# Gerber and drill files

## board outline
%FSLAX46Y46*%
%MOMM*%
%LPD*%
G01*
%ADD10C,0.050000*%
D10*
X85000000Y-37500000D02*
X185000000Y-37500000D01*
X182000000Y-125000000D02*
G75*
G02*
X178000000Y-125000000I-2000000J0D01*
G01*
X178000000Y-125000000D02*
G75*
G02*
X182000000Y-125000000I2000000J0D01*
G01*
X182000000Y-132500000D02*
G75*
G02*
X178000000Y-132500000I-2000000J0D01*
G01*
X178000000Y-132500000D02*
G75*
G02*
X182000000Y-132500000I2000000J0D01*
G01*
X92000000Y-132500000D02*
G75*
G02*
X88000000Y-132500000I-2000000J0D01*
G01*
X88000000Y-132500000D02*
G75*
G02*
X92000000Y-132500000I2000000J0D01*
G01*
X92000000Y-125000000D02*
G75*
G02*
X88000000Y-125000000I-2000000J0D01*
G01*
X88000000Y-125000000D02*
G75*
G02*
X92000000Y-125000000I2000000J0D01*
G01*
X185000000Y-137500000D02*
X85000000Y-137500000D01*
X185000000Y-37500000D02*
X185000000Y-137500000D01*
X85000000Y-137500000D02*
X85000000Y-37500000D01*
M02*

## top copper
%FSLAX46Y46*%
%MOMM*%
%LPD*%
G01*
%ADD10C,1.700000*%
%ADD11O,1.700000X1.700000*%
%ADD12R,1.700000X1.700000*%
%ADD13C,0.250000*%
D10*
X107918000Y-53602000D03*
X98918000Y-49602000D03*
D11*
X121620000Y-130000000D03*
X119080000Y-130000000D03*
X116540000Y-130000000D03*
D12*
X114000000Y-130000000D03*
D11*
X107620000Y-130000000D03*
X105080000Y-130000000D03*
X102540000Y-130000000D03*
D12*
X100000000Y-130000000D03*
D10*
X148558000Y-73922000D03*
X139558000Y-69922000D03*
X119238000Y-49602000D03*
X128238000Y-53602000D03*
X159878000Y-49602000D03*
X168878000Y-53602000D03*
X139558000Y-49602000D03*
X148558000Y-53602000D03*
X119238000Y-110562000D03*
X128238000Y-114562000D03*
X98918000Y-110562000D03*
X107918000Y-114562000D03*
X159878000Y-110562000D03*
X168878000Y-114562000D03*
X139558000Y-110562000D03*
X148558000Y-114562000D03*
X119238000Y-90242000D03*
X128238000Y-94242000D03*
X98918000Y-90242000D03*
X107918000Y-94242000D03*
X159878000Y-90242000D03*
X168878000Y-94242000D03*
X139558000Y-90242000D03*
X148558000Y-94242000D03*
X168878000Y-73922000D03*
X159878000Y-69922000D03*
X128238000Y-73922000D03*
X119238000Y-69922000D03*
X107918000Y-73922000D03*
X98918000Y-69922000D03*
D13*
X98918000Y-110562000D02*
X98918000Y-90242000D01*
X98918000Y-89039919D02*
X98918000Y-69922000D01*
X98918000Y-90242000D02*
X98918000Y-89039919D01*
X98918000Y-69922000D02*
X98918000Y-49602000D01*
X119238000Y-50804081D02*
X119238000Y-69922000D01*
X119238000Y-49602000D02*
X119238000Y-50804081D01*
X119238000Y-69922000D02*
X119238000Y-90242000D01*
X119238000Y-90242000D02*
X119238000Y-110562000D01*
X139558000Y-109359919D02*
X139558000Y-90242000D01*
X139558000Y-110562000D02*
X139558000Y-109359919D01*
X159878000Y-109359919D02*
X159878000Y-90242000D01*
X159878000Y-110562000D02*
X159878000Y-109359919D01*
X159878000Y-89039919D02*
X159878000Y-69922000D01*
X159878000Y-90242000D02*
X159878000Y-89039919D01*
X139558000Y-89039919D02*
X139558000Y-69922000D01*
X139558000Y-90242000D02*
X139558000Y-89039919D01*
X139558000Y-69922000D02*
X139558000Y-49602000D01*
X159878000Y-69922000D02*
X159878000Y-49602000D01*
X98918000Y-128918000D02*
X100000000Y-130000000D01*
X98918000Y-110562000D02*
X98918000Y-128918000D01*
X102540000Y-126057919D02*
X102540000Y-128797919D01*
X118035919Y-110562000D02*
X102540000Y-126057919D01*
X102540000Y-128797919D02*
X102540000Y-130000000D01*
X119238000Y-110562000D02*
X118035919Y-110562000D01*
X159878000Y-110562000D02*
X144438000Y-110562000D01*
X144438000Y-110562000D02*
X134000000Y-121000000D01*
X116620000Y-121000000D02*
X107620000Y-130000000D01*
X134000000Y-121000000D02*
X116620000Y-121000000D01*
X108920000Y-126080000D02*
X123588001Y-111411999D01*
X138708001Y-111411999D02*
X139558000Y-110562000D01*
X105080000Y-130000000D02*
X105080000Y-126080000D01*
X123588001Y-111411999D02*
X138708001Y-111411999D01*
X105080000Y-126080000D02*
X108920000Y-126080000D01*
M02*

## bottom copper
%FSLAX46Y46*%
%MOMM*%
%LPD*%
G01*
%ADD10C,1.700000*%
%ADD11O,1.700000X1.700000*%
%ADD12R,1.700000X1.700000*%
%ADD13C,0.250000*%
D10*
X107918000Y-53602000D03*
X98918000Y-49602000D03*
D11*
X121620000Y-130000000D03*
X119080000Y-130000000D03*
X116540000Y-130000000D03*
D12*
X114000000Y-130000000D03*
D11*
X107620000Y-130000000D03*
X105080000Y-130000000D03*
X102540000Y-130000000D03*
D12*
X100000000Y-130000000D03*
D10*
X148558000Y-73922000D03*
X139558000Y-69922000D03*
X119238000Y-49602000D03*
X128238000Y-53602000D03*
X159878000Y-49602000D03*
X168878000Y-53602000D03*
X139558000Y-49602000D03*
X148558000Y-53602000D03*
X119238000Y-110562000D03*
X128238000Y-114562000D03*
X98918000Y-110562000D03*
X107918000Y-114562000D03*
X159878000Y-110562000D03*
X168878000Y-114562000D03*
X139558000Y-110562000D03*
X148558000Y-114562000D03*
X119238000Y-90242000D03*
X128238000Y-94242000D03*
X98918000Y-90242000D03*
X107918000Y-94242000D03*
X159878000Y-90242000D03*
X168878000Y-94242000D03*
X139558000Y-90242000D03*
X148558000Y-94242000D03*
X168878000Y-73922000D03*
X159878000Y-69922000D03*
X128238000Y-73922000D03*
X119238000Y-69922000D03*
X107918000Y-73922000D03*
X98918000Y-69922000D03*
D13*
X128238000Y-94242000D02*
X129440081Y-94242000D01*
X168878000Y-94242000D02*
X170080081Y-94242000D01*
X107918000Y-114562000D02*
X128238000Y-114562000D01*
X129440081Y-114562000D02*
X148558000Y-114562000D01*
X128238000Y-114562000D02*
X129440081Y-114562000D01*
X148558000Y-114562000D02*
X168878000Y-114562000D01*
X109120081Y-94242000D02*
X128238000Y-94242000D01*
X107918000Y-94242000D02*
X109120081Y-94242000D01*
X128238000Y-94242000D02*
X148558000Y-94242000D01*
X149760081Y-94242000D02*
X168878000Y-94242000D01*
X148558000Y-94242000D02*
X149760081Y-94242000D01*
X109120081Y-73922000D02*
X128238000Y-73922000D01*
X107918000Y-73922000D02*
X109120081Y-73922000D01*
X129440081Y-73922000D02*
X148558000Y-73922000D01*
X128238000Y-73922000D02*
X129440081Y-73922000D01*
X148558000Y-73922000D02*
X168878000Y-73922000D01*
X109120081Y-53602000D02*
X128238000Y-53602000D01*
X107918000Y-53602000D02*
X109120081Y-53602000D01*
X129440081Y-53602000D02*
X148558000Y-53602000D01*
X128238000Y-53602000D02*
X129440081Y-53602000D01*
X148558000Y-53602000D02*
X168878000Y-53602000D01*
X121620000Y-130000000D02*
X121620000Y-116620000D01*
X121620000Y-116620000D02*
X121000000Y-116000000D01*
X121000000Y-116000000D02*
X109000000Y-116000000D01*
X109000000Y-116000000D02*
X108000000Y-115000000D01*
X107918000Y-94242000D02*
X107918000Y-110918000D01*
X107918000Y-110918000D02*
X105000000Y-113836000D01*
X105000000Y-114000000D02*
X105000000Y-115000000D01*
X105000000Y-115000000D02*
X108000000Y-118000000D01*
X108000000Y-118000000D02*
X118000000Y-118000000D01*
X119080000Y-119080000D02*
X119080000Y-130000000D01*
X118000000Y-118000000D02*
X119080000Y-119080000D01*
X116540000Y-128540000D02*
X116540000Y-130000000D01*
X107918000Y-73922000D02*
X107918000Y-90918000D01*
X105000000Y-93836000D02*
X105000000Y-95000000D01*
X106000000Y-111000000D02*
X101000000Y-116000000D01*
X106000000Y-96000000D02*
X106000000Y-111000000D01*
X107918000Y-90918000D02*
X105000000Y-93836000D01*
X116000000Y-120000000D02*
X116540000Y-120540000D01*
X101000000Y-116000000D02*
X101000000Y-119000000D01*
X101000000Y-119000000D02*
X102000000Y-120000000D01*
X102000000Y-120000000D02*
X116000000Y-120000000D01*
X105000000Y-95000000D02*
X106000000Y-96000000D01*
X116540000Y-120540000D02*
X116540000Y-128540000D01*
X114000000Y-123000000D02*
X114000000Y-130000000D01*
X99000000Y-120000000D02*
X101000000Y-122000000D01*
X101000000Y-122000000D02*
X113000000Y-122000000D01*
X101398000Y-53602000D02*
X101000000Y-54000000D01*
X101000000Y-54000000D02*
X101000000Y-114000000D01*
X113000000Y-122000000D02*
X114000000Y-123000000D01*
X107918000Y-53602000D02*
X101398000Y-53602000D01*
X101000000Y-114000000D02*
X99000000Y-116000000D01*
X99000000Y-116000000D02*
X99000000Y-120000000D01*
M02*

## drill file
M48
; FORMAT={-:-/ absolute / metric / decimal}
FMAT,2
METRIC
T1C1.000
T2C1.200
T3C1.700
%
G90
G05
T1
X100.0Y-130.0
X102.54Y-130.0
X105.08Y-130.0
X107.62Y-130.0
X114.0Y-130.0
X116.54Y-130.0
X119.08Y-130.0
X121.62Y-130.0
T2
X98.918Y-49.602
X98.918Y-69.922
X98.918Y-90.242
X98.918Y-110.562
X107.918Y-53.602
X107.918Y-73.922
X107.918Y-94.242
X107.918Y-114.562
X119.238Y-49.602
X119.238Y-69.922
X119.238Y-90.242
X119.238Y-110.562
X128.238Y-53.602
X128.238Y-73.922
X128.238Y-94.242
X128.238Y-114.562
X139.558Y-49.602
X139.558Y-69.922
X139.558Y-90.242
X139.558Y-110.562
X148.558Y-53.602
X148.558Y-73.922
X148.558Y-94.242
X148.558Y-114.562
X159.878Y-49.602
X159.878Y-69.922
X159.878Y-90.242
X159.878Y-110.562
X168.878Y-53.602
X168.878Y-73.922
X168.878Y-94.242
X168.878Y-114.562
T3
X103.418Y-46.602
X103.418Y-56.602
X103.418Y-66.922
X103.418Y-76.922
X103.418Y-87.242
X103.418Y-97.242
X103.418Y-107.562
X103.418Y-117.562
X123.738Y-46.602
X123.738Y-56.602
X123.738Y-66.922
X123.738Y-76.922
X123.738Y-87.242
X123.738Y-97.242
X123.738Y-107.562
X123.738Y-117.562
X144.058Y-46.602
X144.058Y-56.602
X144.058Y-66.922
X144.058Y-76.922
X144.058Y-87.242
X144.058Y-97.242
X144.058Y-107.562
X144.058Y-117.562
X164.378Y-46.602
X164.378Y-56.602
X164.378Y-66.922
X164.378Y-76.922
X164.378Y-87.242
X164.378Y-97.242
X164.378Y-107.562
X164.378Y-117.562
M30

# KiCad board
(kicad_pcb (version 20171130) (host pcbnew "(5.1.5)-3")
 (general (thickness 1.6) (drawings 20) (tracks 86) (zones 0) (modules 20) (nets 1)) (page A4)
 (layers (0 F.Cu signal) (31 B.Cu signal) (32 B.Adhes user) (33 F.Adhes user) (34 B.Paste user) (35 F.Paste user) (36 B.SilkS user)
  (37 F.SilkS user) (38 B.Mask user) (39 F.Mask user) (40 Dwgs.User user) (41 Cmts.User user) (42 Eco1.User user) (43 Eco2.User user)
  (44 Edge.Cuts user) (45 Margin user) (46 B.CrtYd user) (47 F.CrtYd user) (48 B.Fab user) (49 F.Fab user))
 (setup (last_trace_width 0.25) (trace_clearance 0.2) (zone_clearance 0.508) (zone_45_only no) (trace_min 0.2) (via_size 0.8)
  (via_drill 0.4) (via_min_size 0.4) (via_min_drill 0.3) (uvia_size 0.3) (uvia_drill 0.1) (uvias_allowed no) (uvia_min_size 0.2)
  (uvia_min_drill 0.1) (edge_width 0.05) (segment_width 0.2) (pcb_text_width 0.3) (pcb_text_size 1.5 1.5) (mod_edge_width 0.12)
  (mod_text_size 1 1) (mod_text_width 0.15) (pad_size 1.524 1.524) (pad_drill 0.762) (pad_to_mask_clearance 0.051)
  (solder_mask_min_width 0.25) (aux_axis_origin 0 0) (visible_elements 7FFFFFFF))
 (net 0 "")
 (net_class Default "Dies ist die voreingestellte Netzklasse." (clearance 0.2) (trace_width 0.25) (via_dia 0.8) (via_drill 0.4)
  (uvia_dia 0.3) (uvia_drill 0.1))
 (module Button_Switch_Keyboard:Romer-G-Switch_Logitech (layer F.Cu) (at 103.418 51.602)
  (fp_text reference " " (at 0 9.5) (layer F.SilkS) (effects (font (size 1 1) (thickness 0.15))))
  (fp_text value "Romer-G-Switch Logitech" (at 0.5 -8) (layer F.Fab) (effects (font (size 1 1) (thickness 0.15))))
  (pad "" np_thru_hole circle (at 0 5) (size 1.7 1.7) (drill 1.7) (layers *.Cu *.Mask))
  (pad "" np_thru_hole circle (at 0 -5) (size 1.7 1.7) (drill 1.7) (layers *.Cu *.Mask))
  (pad 2 thru_hole circle (at 4.5 2) (size 1.7 1.7) (drill 1.2) (layers *.Cu *.Mask))
  (pad 1 thru_hole circle (at -4.5 -2) (size 1.7 1.7) (drill 1.2) (layers *.Cu *.Mask)))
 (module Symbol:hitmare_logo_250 (layer B.Cu) (at 134 82 180)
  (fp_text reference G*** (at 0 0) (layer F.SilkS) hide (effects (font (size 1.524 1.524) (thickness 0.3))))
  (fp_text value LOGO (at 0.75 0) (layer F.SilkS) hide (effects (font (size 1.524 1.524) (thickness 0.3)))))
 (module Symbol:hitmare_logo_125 (layer F.Cu) (at 180 46)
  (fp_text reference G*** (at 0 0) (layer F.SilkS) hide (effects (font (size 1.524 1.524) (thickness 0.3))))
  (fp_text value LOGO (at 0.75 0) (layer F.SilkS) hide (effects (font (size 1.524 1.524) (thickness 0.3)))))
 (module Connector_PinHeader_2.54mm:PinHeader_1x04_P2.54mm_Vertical (layer F.Cu) (at 114 130 90)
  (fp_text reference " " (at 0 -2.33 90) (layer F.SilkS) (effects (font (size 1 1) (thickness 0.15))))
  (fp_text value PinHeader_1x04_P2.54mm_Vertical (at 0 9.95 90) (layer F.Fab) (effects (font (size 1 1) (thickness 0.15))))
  (pad 4 thru_hole oval (at 0 7.62 90) (size 1.7 1.7) (drill 1) (layers *.Cu *.Mask))
  (pad 3 thru_hole oval (at 0 5.08 90) (size 1.7 1.7) (drill 1) (layers *.Cu *.Mask))
  (pad 2 thru_hole oval (at 0 2.54 90) (size 1.7 1.7) (drill 1) (layers *.Cu *.Mask))
  (pad 1 thru_hole rect (at 0 0 90) (size 1.7 1.7) (drill 1) (layers *.Cu *.Mask)))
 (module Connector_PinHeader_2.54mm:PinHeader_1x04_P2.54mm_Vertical (layer F.Cu) (at 100 130 90)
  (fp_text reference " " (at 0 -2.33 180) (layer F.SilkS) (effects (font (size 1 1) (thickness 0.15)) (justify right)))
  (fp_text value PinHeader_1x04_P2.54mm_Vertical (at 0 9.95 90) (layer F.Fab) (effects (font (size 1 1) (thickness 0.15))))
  (pad 4 thru_hole oval (at 0 7.62 90) (size 1.7 1.7) (drill 1) (layers *.Cu *.Mask))
  (pad 3 thru_hole oval (at 0 5.08 90) (size 1.7 1.7) (drill 1) (layers *.Cu *.Mask))
  (pad 2 thru_hole oval (at 0 2.54 90) (size 1.7 1.7) (drill 1) (layers *.Cu *.Mask))
  (pad 1 thru_hole rect (at 0 0 90) (size 1.7 1.7) (drill 1) (layers *.Cu *.Mask)))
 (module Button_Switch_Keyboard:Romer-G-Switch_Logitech (layer F.Cu) (at 144.058 71.922)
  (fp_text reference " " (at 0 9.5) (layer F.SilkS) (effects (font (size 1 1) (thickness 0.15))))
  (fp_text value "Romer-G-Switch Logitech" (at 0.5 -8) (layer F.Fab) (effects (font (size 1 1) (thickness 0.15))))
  (pad "" np_thru_hole circle (at 0 5) (size 1.7 1.7) (drill 1.7) (layers *.Cu *.Mask))
  (pad "" np_thru_hole circle (at 0 -5) (size 1.7 1.7) (drill 1.7) (layers *.Cu *.Mask))
  (pad 2 thru_hole circle (at 4.5 2) (size 1.7 1.7) (drill 1.2) (layers *.Cu *.Mask))
  (pad 1 thru_hole circle (at -4.5 -2) (size 1.7 1.7) (drill 1.2) (layers *.Cu *.Mask)))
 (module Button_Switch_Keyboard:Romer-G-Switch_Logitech (layer F.Cu) (at 123.738 51.602)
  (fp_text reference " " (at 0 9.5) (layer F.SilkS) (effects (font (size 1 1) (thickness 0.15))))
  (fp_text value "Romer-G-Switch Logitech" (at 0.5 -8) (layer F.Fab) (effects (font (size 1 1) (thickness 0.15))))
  (pad 1 thru_hole circle (at -4.5 -2) (size 1.7 1.7) (drill 1.2) (layers *.Cu *.Mask))
  (pad 2 thru_hole circle (at 4.5 2) (size 1.7 1.7) (drill 1.2) (layers *.Cu *.Mask))
  (pad "" np_thru_hole circle (at 0 -5) (size 1.7 1.7) (drill 1.7) (layers *.Cu *.Mask))
  (pad "" np_thru_hole circle (at 0 5) (size 1.7 1.7) (drill 1.7) (layers *.Cu *.Mask)))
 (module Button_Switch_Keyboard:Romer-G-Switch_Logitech (layer F.Cu) (at 164.378 51.602)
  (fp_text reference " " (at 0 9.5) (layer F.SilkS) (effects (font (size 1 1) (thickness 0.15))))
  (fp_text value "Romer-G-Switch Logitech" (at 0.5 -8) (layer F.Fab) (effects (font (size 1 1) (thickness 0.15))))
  (pad 1 thru_hole circle (at -4.5 -2) (size 1.7 1.7) (drill 1.2) (layers *.Cu *.Mask))
  (pad 2 thru_hole circle (at 4.5 2) (size 1.7 1.7) (drill 1.2) (layers *.Cu *.Mask))
  (pad "" np_thru_hole circle (at 0 -5) (size 1.7 1.7) (drill 1.7) (layers *.Cu *.Mask))
  (pad "" np_thru_hole circle (at 0 5) (size 1.7 1.7) (drill 1.7) (layers *.Cu *.Mask)))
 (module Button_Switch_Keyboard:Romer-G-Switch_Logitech (layer F.Cu) (at 144.058 51.602)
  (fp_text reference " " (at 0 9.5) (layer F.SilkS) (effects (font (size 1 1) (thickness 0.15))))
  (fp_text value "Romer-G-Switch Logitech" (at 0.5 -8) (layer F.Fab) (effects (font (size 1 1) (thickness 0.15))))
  (pad 1 thru_hole circle (at -4.5 -2) (size 1.7 1.7) (drill 1.2) (layers *.Cu *.Mask))
  (pad 2 thru_hole circle (at 4.5 2) (size 1.7 1.7) (drill 1.2) (layers *.Cu *.Mask))
  (pad "" np_thru_hole circle (at 0 -5) (size 1.7 1.7) (drill 1.7) (layers *.Cu *.Mask))
  (pad "" np_thru_hole circle (at 0 5) (size 1.7 1.7) (drill 1.7) (layers *.Cu *.Mask)))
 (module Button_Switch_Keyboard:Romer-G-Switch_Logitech (layer F.Cu) (at 123.738 112.562)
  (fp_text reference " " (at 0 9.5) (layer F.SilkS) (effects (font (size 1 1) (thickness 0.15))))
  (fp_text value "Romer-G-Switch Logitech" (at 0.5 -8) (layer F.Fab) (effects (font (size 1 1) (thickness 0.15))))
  (pad 1 thru_hole circle (at -4.5 -2) (size 1.7 1.7) (drill 1.2) (layers *.Cu *.Mask))
  (pad 2 thru_hole circle (at 4.5 2) (size 1.7 1.7) (drill 1.2) (layers *.Cu *.Mask))
  (pad "" np_thru_hole circle (at 0 -5) (size 1.7 1.7) (drill 1.7) (layers *.Cu *.Mask))
  (pad "" np_thru_hole circle (at 0 5) (size 1.7 1.7) (drill 1.7) (layers *.Cu *.Mask)))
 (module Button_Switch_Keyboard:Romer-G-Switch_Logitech (layer F.Cu) (at 103.418 112.562)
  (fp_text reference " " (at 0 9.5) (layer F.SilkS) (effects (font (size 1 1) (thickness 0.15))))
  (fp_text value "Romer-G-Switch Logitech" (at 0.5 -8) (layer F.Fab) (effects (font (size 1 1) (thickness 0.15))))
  (pad 1 thru_hole circle (at -4.5 -2) (size 1.7 1.7) (drill 1.2) (layers *.Cu *.Mask))
  (pad 2 thru_hole circle (at 4.5 2) (size 1.7 1.7) (drill 1.2) (layers *.Cu *.Mask))
  (pad "" np_thru_hole circle (at 0 -5) (size 1.7 1.7) (drill 1.7) (layers *.Cu *.Mask))
  (pad "" np_thru_hole circle (at 0 5) (size 1.7 1.7) (drill 1.7) (layers *.Cu *.Mask)))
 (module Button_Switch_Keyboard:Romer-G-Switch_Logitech (layer F.Cu) (at 164.378 112.562)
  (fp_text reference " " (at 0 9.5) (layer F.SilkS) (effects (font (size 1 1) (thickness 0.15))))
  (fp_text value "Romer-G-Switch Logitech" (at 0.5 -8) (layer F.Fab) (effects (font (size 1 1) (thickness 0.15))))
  (pad 1 thru_hole circle (at -4.5 -2) (size 1.7 1.7) (drill 1.2) (layers *.Cu *.Mask))
  (pad 2 thru_hole circle (at 4.5 2) (size 1.7 1.7) (drill 1.2) (layers *.Cu *.Mask))
  (pad "" np_thru_hole circle (at 0 -5) (size 1.7 1.7) (drill 1.7) (layers *.Cu *.Mask))
  (pad "" np_thru_hole circle (at 0 5) (size 1.7 1.7) (drill 1.7) (layers *.Cu *.Mask)))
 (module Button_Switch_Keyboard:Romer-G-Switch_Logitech (layer F.Cu) (at 144.058 112.562)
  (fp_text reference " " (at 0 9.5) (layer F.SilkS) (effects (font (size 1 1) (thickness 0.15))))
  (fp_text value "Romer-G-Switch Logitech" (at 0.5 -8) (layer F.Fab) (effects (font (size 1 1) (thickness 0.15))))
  (pad 1 thru_hole circle (at -4.5 -2) (size 1.7 1.7) (drill 1.2) (layers *.Cu *.Mask))
  (pad 2 thru_hole circle (at 4.5 2) (size 1.7 1.7) (drill 1.2) (layers *.Cu *.Mask))
  (pad "" np_thru_hole circle (at 0 -5) (size 1.7 1.7) (drill 1.7) (layers *.Cu *.Mask))
  (pad "" np_thru_hole circle (at 0 5) (size 1.7 1.7) (drill 1.7) (layers *.Cu *.Mask)))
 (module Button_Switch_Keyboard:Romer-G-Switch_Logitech (layer F.Cu) (at 123.738 92.242)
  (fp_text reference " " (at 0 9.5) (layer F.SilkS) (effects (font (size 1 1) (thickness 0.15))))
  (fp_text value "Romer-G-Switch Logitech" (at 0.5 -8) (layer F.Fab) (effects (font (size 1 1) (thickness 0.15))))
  (pad 1 thru_hole circle (at -4.5 -2) (size 1.7 1.7) (drill 1.2) (layers *.Cu *.Mask))
  (pad 2 thru_hole circle (at 4.5 2) (size 1.7 1.7) (drill 1.2) (layers *.Cu *.Mask))
  (pad "" np_thru_hole circle (at 0 -5) (size 1.7 1.7) (drill 1.7) (layers *.Cu *.Mask))
  (pad "" np_thru_hole circle (at 0 5) (size 1.7 1.7) (drill 1.7) (layers *.Cu *.Mask)))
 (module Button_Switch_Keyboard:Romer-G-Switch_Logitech (layer F.Cu) (at 103.418 92.242)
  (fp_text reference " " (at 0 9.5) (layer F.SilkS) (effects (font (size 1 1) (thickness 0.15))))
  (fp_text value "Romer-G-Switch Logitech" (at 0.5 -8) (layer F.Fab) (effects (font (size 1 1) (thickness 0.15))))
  (pad 1 thru_hole circle (at -4.5 -2) (size 1.7 1.7) (drill 1.2) (layers *.Cu *.Mask))
  (pad 2 thru_hole circle (at 4.5 2) (size 1.7 1.7) (drill 1.2) (layers *.Cu *.Mask))
  (pad "" np_thru_hole circle (at 0 -5) (size 1.7 1.7) (drill 1.7) (layers *.Cu *.Mask))
  (pad "" np_thru_hole circle (at 0 5) (size 1.7 1.7) (drill 1.7) (layers *.Cu *.Mask)))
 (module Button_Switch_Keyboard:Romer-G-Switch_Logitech (layer F.Cu) (at 164.378 92.242)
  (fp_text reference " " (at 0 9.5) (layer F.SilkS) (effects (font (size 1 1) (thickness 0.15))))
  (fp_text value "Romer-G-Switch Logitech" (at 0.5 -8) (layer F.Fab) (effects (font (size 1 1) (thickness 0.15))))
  (pad 1 thru_hole circle (at -4.5 -2) (size 1.7 1.7) (drill 1.2) (layers *.Cu *.Mask))
  (pad 2 thru_hole circle (at 4.5 2) (size 1.7 1.7) (drill 1.2) (layers *.Cu *.Mask))
  (pad "" np_thru_hole circle (at 0 -5) (size 1.7 1.7) (drill 1.7) (layers *.Cu *.Mask))
  (pad "" np_thru_hole circle (at 0 5) (size 1.7 1.7) (drill 1.7) (layers *.Cu *.Mask)))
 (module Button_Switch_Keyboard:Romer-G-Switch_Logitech (layer F.Cu) (at 144.058 92.242)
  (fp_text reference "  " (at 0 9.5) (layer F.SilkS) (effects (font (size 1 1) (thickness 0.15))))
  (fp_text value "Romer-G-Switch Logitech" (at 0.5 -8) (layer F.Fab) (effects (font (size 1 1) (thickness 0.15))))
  (pad 1 thru_hole circle (at -4.5 -2) (size 1.7 1.7) (drill 1.2) (layers *.Cu *.Mask))
  (pad 2 thru_hole circle (at 4.5 2) (size 1.7 1.7) (drill 1.2) (layers *.Cu *.Mask))
  (pad "" np_thru_hole circle (at 0 -5) (size 1.7 1.7) (drill 1.7) (layers *.Cu *.Mask))
  (pad "" np_thru_hole circle (at 0 5) (size 1.7 1.7) (drill 1.7) (layers *.Cu *.Mask)))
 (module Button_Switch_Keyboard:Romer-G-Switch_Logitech (layer F.Cu) (at 164.378 71.922)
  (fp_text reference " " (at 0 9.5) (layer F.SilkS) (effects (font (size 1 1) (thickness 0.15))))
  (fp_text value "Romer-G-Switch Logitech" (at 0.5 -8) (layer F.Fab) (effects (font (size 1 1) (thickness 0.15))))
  (pad "" np_thru_hole circle (at 0 5) (size 1.7 1.7) (drill 1.7) (layers *.Cu *.Mask))
  (pad "" np_thru_hole circle (at 0 -5) (size 1.7 1.7) (drill 1.7) (layers *.Cu *.Mask))
  (pad 2 thru_hole circle (at 4.5 2) (size 1.7 1.7) (drill 1.2) (layers *.Cu *.Mask))
  (pad 1 thru_hole circle (at -4.5 -2) (size 1.7 1.7) (drill 1.2) (layers *.Cu *.Mask)))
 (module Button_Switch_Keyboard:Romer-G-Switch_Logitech (layer F.Cu) (at 123.738 71.922)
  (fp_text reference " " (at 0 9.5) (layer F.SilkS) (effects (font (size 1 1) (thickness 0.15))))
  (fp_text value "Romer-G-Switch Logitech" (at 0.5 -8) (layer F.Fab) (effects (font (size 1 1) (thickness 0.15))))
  (pad "" np_thru_hole circle (at 0 5) (size 1.7 1.7) (drill 1.7) (layers *.Cu *.Mask))
  (pad "" np_thru_hole circle (at 0 -5) (size 1.7 1.7) (drill 1.7) (layers *.Cu *.Mask))
  (pad 2 thru_hole circle (at 4.5 2) (size 1.7 1.7) (drill 1.2) (layers *.Cu *.Mask))
  (pad 1 thru_hole circle (at -4.5 -2) (size 1.7 1.7) (drill 1.2) (layers *.Cu *.Mask)))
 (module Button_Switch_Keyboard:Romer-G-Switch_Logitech (layer F.Cu) (at 103.418 71.922)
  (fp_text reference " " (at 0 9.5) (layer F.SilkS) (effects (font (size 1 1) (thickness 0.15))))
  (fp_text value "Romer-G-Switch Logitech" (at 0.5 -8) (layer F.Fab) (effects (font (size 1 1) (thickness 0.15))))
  (pad "" np_thru_hole circle (at 0 5) (size 1.7 1.7) (drill 1.7) (layers *.Cu *.Mask))
  (pad "" np_thru_hole circle (at 0 -5) (size 1.7 1.7) (drill 1.7) (layers *.Cu *.Mask))
  (pad 2 thru_hole circle (at 4.5 2) (size 1.7 1.7) (drill 1.2) (layers *.Cu *.Mask))
  (pad 1 thru_hole circle (at -4.5 -2) (size 1.7 1.7) (drill 1.2) (layers *.Cu *.Mask)))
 (gr_line (start 85 37.5) (end 185 37.5) (layer Edge.Cuts) (width 0.05))
 (gr_circle (center 180 125) (end 182 125) (layer Edge.Cuts) (width 0.05))
 (gr_circle (center 180 132.5) (end 182 132.5) (layer Edge.Cuts) (width 0.05))
 (gr_circle (center 90 132.5) (end 92 132.5) (layer Edge.Cuts) (width 0.05))
 (gr_circle (center 90 125) (end 92 125) (layer Edge.Cuts) (width 0.05))
 (gr_line (start 185 137.5) (end 85 137.5) (layer Edge.Cuts) (width 0.05))
 (gr_line (start 185 37.5) (end 185 137.5) (layer Edge.Cuts) (width 0.05))
 (gr_line (start 85 137.5) (end 85 37.5) (layer Edge.Cuts) (width 0.05))
 (segment (start 128.238 94.242) (end 129.440081 94.242) (width 0.25) (layer B.Cu) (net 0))
 (segment (start 168.878 94.242) (end 170.080081 94.242) (width 0.25) (layer B.Cu) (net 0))
 (segment (start 98.918 110.562) (end 98.918 90.242) (width 0.25) (layer F.Cu) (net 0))
 (segment (start 98.918 89.039919) (end 98.918 69.922) (width 0.25) (layer F.Cu) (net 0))
 (segment (start 98.918 90.242) (end 98.918 89.039919) (width 0.25) (layer F.Cu) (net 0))
 (segment (start 98.918 69.922) (end 98.918 49.602) (width 0.25) (layer F.Cu) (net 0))
 (segment (start 119.238 50.804081) (end 119.238 69.922) (width 0.25) (layer F.Cu) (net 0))
 (segment (start 119.238 49.602) (end 119.238 50.804081) (width 0.25) (layer F.Cu) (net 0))
 (segment (start 119.238 69.922) (end 119.238 90.242) (width 0.25) (layer F.Cu) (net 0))
 (segment (start 119.238 90.242) (end 119.238 110.562) (width 0.25) (layer F.Cu) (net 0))
 (segment (start 139.558 109.359919) (end 139.558 90.242) (width 0.25) (layer F.Cu) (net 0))
 (segment (start 139.558 110.562) (end 139.558 109.359919) (width 0.25) (layer F.Cu) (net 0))
 (segment (start 159.878 109.359919) (end 159.878 90.242) (width 0.25) (layer F.Cu) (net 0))
 (segment (start 159.878 110.562) (end 159.878 109.359919) (width 0.25) (layer F.Cu) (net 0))
 (segment (start 159.878 89.039919) (end 159.878 69.922) (width 0.25) (layer F.Cu) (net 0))
 (segment (start 159.878 90.242) (end 159.878 89.039919) (width 0.25) (layer F.Cu) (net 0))
 (segment (start 139.558 89.039919) (end 139.558 69.922) (width 0.25) (layer F.Cu) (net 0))
 (segment (start 139.558 90.242) (end 139.558 89.039919) (width 0.25) (layer F.Cu) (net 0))
 (segment (start 139.558 69.922) (end 139.558 49.602) (width 0.25) (layer F.Cu) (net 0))
 (segment (start 159.878 69.922) (end 159.878 49.602) (width 0.25) (layer F.Cu) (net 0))
 (segment (start 107.918 114.562) (end 128.238 114.562) (width 0.25) (layer B.Cu) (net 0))
 (segment (start 129.440081 114.562) (end 148.558 114.562) (width 0.25) (layer B.Cu) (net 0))
 (segment (start 128.238 114.562) (end 129.440081 114.562) (width 0.25) (layer B.Cu) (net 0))
 (segment (start 148.558 114.562) (end 168.878 114.562) (width 0.25) (layer B.Cu) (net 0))
 (segment (start 109.120081 94.242) (end 128.238 94.242) (width 0.25) (layer B.Cu) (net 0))
 (segment (start 107.918 94.242) (end 109.120081 94.242) (width 0.25) (layer B.Cu) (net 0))
 (segment (start 128.238 94.242) (end 148.558 94.242) (width 0.25) (layer B.Cu) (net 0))
 (segment (start 149.760081 94.242) (end 168.878 94.242) (width 0.25) (layer B.Cu) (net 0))
 (segment (start 148.558 94.242) (end 149.760081 94.242) (width 0.25) (layer B.Cu) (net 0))
 (segment (start 109.120081 73.922) (end 128.238 73.922) (width 0.25) (layer B.Cu) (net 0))
 (segment (start 107.918 73.922) (end 109.120081 73.922) (width 0.25) (layer B.Cu) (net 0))
 (segment (start 129.440081 73.922) (end 148.558 73.922) (width 0.25) (layer B.Cu) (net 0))
 (segment (start 128.238 73.922) (end 129.440081 73.922) (width 0.25) (layer B.Cu) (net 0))
 (segment (start 148.558 73.922) (end 168.878 73.922) (width 0.25) (layer B.Cu) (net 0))
 (segment (start 109.120081 53.602) (end 128.238 53.602) (width 0.25) (layer B.Cu) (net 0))
 (segment (start 107.918 53.602) (end 109.120081 53.602) (width 0.25) (layer B.Cu) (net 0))
 (segment (start 129.440081 53.602) (end 148.558 53.602) (width 0.25) (layer B.Cu) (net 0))
 (segment (start 128.238 53.602) (end 129.440081 53.602) (width 0.25) (layer B.Cu) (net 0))
 (segment (start 148.558 53.602) (end 168.878 53.602) (width 0.25) (layer B.Cu) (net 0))
 (segment (start 98.918 128.918) (end 100 130) (width 0.25) (layer F.Cu) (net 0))
 (segment (start 98.918 110.562) (end 98.918 128.918) (width 0.25) (layer F.Cu) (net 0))
 (segment (start 102.54 126.057919) (end 102.54 128.797919) (width 0.25) (layer F.Cu) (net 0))
 (segment (start 118.035919 110.562) (end 102.54 126.057919) (width 0.25) (layer F.Cu) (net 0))
 (segment (start 102.54 128.797919) (end 102.54 130) (width 0.25) (layer F.Cu) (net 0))
 (segment (start 119.238 110.562) (end 118.035919 110.562) (width 0.25) (layer F.Cu) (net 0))
 (segment (start 159.878 110.562) (end 144.438 110.562) (width 0.25) (layer F.Cu) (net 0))
 (segment (start 144.438 110.562) (end 134 121) (width 0.25) (layer F.Cu) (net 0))
 (segment (start 116.62 121) (end 107.62 130) (width 0.25) (layer F.Cu) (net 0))
 (segment (start 134 121) (end 116.62 121) (width 0.25) (layer F.Cu) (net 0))
 (segment (start 108.92 126.08) (end 123.588001 111.411999) (width 0.25) (layer F.Cu) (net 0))
 (segment (start 138.708001 111.411999) (end 139.558 110.562) (width 0.25) (layer F.Cu) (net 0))
 (segment (start 105.08 130) (end 105.08 126.08) (width 0.25) (layer F.Cu) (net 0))
 (segment (start 123.588001 111.411999) (end 138.708001 111.411999) (width 0.25) (layer F.Cu) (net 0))
 (segment (start 105.08 126.08) (end 108.92 126.08) (width 0.25) (layer F.Cu) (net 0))
 (segment (start 121.62 130) (end 121.62 116.62) (width 0.25) (layer B.Cu) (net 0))
 (segment (start 121.62 116.62) (end 121 116) (width 0.25) (layer B.Cu) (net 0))
 (segment (start 121 116) (end 109 116) (width 0.25) (layer B.Cu) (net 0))
 (segment (start 109 116) (end 108 115) (width 0.25) (layer B.Cu) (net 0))
 (segment (start 107.918 94.242) (end 107.918 110.918) (width 0.25) (layer B.Cu) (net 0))
 (segment (start 107.918 110.918) (end 105 113.836) (width 0.25) (layer B.Cu) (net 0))
 (segment (start 105 114) (end 105 115) (width 0.25) (layer B.Cu) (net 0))
 (segment (start 105 115) (end 108 118) (width 0.25) (layer B.Cu) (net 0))
 (segment (start 108 118) (end 118 118) (width 0.25) (layer B.Cu) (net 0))
 (segment (start 119.08 119.08) (end 119.08 130) (width 0.25) (layer B.Cu) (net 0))
 (segment (start 118 118) (end 119.08 119.08) (width 0.25) (layer B.Cu) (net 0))
 (segment (start 116.54 128.54) (end 116.54 130) (width 0.25) (layer B.Cu) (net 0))
 (segment (start 107.918 73.922) (end 107.918 90.918) (width 0.25) (layer B.Cu) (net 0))
 (segment (start 105 93.836) (end 105 95) (width 0.25) (layer B.Cu) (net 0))
 (segment (start 106 111) (end 101 116) (width 0.25) (layer B.Cu) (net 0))
 (segment (start 106 96) (end 106 111) (width 0.25) (layer B.Cu) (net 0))
 (segment (start 107.918 90.918) (end 105 93.836) (width 0.25) (layer B.Cu) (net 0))
 (segment (start 116 120) (end 116.54 120.54) (width 0.25) (layer B.Cu) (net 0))
 (segment (start 101 116) (end 101 119) (width 0.25) (layer B.Cu) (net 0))
 (segment (start 101 119) (end 102 120) (width 0.25) (layer B.Cu) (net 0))
 (segment (start 102 120) (end 116 120) (width 0.25) (layer B.Cu) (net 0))
 (segment (start 105 95) (end 106 96) (width 0.25) (layer B.Cu) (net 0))
 (segment (start 116.54 120.54) (end 116.54 128.54) (width 0.25) (layer B.Cu) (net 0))
 (segment (start 114 123) (end 114 130) (width 0.25) (layer B.Cu) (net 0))
 (segment (start 99 120) (end 101 122) (width 0.25) (layer B.Cu) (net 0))
 (segment (start 101 122) (end 113 122) (width 0.25) (layer B.Cu) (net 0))
 (segment (start 101.398 53.602) (end 101 54) (width 0.25) (layer B.Cu) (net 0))
 (segment (start 101 54) (end 101 114) (width 0.25) (layer B.Cu) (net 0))
 (segment (start 113 122) (end 114 123) (width 0.25) (layer B.Cu) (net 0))
 (segment (start 107.918 53.602) (end 101.398 53.602) (width 0.25) (layer B.Cu) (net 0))
 (segment (start 101 114) (end 99 116) (width 0.25) (layer B.Cu) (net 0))
 (segment (start 99 116) (end 99 120) (width 0.25) (layer B.Cu) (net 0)))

